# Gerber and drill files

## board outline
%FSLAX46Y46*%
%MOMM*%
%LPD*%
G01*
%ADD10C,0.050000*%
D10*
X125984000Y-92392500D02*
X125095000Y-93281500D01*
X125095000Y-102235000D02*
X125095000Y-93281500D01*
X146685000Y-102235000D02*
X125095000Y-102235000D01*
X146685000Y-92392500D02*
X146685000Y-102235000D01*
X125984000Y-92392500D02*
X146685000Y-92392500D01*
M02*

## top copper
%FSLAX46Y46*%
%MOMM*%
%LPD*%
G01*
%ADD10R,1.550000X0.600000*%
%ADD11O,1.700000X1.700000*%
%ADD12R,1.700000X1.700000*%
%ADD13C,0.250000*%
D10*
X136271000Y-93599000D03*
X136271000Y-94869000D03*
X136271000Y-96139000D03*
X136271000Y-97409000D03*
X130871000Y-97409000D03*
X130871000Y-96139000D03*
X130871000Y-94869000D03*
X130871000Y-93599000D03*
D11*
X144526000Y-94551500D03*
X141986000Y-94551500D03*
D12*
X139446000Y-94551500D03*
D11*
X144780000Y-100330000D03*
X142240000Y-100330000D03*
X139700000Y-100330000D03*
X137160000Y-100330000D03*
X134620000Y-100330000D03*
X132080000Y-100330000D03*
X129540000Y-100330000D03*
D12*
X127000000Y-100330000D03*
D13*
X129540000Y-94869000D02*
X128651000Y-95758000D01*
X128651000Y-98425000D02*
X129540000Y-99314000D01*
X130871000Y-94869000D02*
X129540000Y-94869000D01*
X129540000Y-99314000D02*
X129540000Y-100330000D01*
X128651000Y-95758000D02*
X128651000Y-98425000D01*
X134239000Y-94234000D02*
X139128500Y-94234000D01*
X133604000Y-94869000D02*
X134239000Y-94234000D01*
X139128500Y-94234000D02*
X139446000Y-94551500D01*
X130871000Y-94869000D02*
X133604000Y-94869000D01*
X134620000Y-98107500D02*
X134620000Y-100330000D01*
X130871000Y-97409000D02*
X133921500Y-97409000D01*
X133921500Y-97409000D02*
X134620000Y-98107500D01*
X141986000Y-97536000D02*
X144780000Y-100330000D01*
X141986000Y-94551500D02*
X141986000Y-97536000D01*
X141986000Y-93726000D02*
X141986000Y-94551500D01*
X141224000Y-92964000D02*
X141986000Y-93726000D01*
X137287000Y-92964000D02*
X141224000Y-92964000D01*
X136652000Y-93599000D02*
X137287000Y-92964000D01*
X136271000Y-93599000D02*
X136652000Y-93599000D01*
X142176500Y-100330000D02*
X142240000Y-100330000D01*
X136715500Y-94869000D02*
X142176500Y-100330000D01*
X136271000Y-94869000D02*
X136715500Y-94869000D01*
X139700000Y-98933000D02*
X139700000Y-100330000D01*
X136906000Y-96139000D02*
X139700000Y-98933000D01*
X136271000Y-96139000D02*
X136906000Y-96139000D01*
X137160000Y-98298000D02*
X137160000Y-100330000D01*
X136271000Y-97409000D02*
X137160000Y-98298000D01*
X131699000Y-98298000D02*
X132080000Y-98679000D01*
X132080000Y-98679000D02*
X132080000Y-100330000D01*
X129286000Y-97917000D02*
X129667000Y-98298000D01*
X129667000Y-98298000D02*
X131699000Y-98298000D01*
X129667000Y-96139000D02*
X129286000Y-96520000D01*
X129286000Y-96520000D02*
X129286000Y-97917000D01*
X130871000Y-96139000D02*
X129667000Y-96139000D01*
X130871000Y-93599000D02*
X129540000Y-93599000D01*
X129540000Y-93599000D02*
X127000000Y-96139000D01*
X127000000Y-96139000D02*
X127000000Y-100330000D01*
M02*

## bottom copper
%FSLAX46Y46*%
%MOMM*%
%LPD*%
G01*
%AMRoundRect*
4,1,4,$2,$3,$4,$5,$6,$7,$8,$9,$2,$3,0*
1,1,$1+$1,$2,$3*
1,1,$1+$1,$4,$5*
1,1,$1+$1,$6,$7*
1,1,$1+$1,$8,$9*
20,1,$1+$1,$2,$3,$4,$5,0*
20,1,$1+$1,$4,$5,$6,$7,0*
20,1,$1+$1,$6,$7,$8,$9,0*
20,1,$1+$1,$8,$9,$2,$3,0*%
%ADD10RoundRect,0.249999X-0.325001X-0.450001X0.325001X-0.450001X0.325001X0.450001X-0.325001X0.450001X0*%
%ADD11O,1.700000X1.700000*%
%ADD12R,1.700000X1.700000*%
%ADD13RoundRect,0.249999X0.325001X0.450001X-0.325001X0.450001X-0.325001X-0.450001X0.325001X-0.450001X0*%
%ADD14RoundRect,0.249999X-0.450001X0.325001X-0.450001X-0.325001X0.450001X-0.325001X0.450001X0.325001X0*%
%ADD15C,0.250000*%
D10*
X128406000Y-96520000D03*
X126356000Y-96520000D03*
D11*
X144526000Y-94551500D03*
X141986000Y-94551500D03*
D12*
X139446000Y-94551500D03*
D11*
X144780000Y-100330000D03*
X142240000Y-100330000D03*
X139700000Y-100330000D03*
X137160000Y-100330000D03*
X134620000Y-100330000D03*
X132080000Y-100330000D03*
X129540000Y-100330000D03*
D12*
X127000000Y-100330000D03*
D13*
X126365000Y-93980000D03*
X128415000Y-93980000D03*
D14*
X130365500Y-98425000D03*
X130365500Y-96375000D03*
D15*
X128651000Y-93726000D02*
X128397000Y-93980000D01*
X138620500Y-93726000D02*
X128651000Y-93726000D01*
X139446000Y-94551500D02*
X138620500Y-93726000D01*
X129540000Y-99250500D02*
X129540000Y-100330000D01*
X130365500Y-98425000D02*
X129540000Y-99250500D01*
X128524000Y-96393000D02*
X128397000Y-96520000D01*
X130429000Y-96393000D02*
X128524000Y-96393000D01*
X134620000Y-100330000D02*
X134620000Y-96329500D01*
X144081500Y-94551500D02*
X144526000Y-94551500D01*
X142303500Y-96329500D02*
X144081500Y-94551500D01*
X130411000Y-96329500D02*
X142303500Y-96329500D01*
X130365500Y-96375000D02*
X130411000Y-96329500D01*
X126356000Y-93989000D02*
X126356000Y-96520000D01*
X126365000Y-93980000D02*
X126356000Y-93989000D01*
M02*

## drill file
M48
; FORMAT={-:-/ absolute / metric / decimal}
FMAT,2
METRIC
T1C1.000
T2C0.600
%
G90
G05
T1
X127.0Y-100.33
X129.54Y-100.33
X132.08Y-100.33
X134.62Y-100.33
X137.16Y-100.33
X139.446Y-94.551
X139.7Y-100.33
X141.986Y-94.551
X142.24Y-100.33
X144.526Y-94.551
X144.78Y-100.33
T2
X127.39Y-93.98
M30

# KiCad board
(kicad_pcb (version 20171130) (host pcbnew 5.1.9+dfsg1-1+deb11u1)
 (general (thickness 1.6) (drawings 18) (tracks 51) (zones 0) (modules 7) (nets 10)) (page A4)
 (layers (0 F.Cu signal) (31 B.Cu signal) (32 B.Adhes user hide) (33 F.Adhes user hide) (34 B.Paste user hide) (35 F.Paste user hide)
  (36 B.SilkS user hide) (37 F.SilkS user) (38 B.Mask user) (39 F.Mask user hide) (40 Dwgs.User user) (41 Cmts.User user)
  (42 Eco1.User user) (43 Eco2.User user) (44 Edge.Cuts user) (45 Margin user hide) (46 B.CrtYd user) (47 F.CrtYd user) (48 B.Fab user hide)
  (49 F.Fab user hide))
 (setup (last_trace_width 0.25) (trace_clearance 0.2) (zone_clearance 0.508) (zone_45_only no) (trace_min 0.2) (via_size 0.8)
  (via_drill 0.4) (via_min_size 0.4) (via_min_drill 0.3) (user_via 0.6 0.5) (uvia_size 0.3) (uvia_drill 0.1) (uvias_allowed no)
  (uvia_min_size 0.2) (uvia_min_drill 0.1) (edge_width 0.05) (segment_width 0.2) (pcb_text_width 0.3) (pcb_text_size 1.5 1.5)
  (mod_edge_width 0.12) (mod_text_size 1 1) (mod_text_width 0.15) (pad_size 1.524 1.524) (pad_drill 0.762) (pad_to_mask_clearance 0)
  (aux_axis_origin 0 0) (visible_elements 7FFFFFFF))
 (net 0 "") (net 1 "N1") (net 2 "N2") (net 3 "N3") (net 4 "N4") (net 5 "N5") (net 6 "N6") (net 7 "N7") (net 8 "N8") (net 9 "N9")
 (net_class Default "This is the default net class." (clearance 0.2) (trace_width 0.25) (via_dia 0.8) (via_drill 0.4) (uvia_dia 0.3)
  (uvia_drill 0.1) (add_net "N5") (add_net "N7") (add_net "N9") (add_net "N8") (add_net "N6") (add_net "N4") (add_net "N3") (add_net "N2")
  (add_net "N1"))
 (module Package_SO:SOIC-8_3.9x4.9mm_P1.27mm (layer F.Cu) (at 133.571 95.504)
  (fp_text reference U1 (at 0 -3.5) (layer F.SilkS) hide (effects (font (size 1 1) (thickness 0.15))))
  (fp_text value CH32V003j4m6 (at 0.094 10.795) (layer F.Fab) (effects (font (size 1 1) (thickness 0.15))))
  (pad 8 smd rect (at 2.7 -1.905) (size 1.55 0.6) (layers F.Cu F.Paste F.Mask) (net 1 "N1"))
  (pad 7 smd rect (at 2.7 -0.635) (size 1.55 0.6) (layers F.Cu F.Paste F.Mask) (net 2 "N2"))
  (pad 6 smd rect (at 2.7 0.635) (size 1.55 0.6) (layers F.Cu F.Paste F.Mask) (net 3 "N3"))
  (pad 5 smd rect (at 2.7 1.905) (size 1.55 0.6) (layers F.Cu F.Paste F.Mask) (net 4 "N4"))
  (pad 4 smd rect (at -2.7 1.905) (size 1.55 0.6) (layers F.Cu F.Paste F.Mask) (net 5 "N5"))
  (pad 3 smd rect (at -2.7 0.635) (size 1.55 0.6) (layers F.Cu F.Paste F.Mask) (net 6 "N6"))
  (pad 2 smd rect (at -2.7 -0.635) (size 1.55 0.6) (layers F.Cu F.Paste F.Mask) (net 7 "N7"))
  (pad 1 smd rect (at -2.7 -1.905) (size 1.55 0.6) (layers F.Cu F.Paste F.Mask) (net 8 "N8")))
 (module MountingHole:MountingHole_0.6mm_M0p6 (layer F.Cu) (at 127.39 93.98)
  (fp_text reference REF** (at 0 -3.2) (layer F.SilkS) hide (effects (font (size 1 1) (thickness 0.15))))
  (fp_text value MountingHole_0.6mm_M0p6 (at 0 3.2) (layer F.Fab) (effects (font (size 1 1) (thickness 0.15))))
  (pad "" np_thru_hole circle (at 0 0) (size 0.6 0.6) (drill 0.6) (layers *.Cu *.Mask)))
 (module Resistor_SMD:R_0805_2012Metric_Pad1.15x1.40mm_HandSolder (layer B.Cu) (at 127.381 96.52)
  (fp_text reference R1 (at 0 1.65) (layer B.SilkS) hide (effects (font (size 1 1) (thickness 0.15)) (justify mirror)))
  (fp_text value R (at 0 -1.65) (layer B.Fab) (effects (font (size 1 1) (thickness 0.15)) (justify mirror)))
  (pad 2 smd roundrect (at 1.025 0) (size 1.15 1.4) (layers B.Cu B.Paste B.Mask) (roundrect_rratio 0.2173904347826087) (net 5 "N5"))
  (pad 1 smd roundrect (at -1.025 0) (size 1.15 1.4) (layers B.Cu B.Paste B.Mask) (roundrect_rratio 0.2173904347826087) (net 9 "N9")))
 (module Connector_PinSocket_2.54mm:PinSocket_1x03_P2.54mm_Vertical (layer F.Cu) (at 139.446 94.5515 90)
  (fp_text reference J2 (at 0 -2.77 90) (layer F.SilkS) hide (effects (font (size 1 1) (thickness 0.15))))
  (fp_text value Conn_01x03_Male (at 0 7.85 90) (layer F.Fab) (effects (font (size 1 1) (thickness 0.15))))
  (pad 3 thru_hole oval (at 0 5.08 90) (size 1.7 1.7) (drill 1) (layers *.Cu *.Mask) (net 5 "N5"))
  (pad 2 thru_hole oval (at 0 2.54 90) (size 1.7 1.7) (drill 1) (layers *.Cu *.Mask) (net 1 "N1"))
  (pad 1 thru_hole rect (at 0 0 90) (size 1.7 1.7) (drill 1) (layers *.Cu *.Mask) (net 7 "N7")))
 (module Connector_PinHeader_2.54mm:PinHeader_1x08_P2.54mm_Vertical (layer F.Cu) (at 127 100.33 90)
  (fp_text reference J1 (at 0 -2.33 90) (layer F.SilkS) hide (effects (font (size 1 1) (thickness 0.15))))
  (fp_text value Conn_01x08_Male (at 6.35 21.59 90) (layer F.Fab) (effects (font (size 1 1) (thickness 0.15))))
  (pad 8 thru_hole oval (at 0 17.78 90) (size 1.7 1.7) (drill 1) (layers *.Cu *.Mask) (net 1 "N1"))
  (pad 7 thru_hole oval (at 0 15.24 90) (size 1.7 1.7) (drill 1) (layers *.Cu *.Mask) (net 2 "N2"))
  (pad 6 thru_hole oval (at 0 12.7 90) (size 1.7 1.7) (drill 1) (layers *.Cu *.Mask) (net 3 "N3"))
  (pad 5 thru_hole oval (at 0 10.16 90) (size 1.7 1.7) (drill 1) (layers *.Cu *.Mask) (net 4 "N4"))
  (pad 4 thru_hole oval (at 0 7.62 90) (size 1.7 1.7) (drill 1) (layers *.Cu *.Mask) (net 5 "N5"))
  (pad 3 thru_hole oval (at 0 5.08 90) (size 1.7 1.7) (drill 1) (layers *.Cu *.Mask) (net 6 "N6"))
  (pad 2 thru_hole oval (at 0 2.54 90) (size 1.7 1.7) (drill 1) (layers *.Cu *.Mask) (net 7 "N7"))
  (pad 1 thru_hole rect (at 0 0 90) (size 1.7 1.7) (drill 1) (layers *.Cu *.Mask) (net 8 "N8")))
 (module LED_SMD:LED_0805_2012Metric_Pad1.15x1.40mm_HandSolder (layer B.Cu) (at 127.39 93.98 180)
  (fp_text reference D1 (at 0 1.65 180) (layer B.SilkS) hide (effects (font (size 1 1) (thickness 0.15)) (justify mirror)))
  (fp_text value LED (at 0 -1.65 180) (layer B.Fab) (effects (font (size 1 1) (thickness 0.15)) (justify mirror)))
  (pad 2 smd roundrect (at 1.025 0 180) (size 1.15 1.4) (layers B.Cu B.Paste B.Mask) (roundrect_rratio 0.2173904347826087) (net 9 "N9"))
  (pad 1 smd roundrect (at -1.025 0 180) (size 1.15 1.4) (layers B.Cu B.Paste B.Mask) (roundrect_rratio 0.2173904347826087) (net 7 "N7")))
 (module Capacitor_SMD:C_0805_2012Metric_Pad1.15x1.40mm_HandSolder (layer B.Cu) (at 130.3655 97.4 270)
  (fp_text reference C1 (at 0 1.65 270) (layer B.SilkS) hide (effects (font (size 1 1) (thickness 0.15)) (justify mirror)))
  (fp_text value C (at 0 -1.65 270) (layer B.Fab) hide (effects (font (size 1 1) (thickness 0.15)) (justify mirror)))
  (pad 2 smd roundrect (at 1.025 0 270) (size 1.15 1.4) (layers B.Cu B.Paste B.Mask) (roundrect_rratio 0.2173904347826087) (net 7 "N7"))
  (pad 1 smd roundrect (at -1.025 0 270) (size 1.15 1.4) (layers B.Cu B.Paste B.Mask) (roundrect_rratio 0.2173904347826087) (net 5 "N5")))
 (gr_line (start 125.984 92.3925) (end 125.095 93.2815) (layer Edge.Cuts) (width 0.05))
 (gr_line (start 125.095 102.235) (end 125.095 93.2815) (layer Edge.Cuts) (width 0.05))
 (gr_line (start 146.685 102.235) (end 125.095 102.235) (layer Edge.Cuts) (width 0.05))
 (gr_line (start 146.685 92.3925) (end 146.685 102.235) (layer Edge.Cuts) (width 0.05))
 (gr_line (start 125.984 92.3925) (end 146.685 92.3925) (layer Edge.Cuts) (width 0.05))
 (segment (start 129.54 94.869) (end 128.651 95.758) (width 0.25) (layer F.Cu) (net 7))
 (segment (start 128.651 98.425) (end 129.54 99.314) (width 0.25) (layer F.Cu) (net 7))
 (segment (start 130.871 94.869) (end 129.54 94.869) (width 0.25) (layer F.Cu) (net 7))
 (segment (start 129.54 99.314) (end 129.54 100.33) (width 0.25) (layer F.Cu) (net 7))
 (segment (start 128.651 95.758) (end 128.651 98.425) (width 0.25) (layer F.Cu) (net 7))
 (segment (start 128.651 93.726) (end 128.397 93.98) (width 0.25) (layer B.Cu) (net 7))
 (segment (start 138.6205 93.726) (end 128.651 93.726) (width 0.25) (layer B.Cu) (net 7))
 (segment (start 139.446 94.5515) (end 138.6205 93.726) (width 0.25) (layer B.Cu) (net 7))
 (segment (start 134.239 94.234) (end 139.1285 94.234) (width 0.25) (layer F.Cu) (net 7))
 (segment (start 133.604 94.869) (end 134.239 94.234) (width 0.25) (layer F.Cu) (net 7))
 (segment (start 139.1285 94.234) (end 139.446 94.5515) (width 0.25) (layer F.Cu) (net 7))
 (segment (start 130.871 94.869) (end 133.604 94.869) (width 0.25) (layer F.Cu) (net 7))
 (segment (start 129.54 99.2505) (end 129.54 100.33) (width 0.25) (layer B.Cu) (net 7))
 (segment (start 130.3655 98.425) (end 129.54 99.2505) (width 0.25) (layer B.Cu) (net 7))
 (segment (start 134.62 98.1075) (end 134.62 100.33) (width 0.25) (layer F.Cu) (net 5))
 (segment (start 130.871 97.409) (end 133.9215 97.409) (width 0.25) (layer F.Cu) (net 5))
 (segment (start 133.9215 97.409) (end 134.62 98.1075) (width 0.25) (layer F.Cu) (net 5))
 (segment (start 128.524 96.393) (end 128.397 96.52) (width 0.25) (layer B.Cu) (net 5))
 (segment (start 130.429 96.393) (end 128.524 96.393) (width 0.25) (layer B.Cu) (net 5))
 (segment (start 134.62 100.33) (end 134.62 96.3295) (width 0.25) (layer B.Cu) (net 5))
 (segment (start 144.0815 94.5515) (end 144.526 94.5515) (width 0.25) (layer B.Cu) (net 5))
 (segment (start 142.3035 96.3295) (end 144.0815 94.5515) (width 0.25) (layer B.Cu) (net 5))
 (segment (start 130.411 96.3295) (end 142.3035 96.3295) (width 0.25) (layer B.Cu) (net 5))
 (segment (start 130.3655 96.375) (end 130.411 96.3295) (width 0.25) (layer B.Cu) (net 5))
 (segment (start 126.356 93.989) (end 126.356 96.52) (width 0.25) (layer B.Cu) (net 9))
 (segment (start 126.365 93.98) (end 126.356 93.989) (width 0.25) (layer B.Cu) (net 9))
 (segment (start 141.986 97.536) (end 144.78 100.33) (width 0.25) (layer F.Cu) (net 1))
 (segment (start 141.986 94.5515) (end 141.986 97.536) (width 0.25) (layer F.Cu) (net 1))
 (segment (start 141.986 93.726) (end 141.986 94.5515) (width 0.25) (layer F.Cu) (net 1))
 (segment (start 141.224 92.964) (end 141.986 93.726) (width 0.25) (layer F.Cu) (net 1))
 (segment (start 137.287 92.964) (end 141.224 92.964) (width 0.25) (layer F.Cu) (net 1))
 (segment (start 136.652 93.599) (end 137.287 92.964) (width 0.25) (layer F.Cu) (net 1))
 (segment (start 136.271 93.599) (end 136.652 93.599) (width 0.25) (layer F.Cu) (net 1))
 (segment (start 142.1765 100.33) (end 142.24 100.33) (width 0.25) (layer F.Cu) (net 2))
 (segment (start 136.7155 94.869) (end 142.1765 100.33) (width 0.25) (layer F.Cu) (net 2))
 (segment (start 136.271 94.869) (end 136.7155 94.869) (width 0.25) (layer F.Cu) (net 2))
 (segment (start 139.7 98.933) (end 139.7 100.33) (width 0.25) (layer F.Cu) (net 3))
 (segment (start 136.906 96.139) (end 139.7 98.933) (width 0.25) (layer F.Cu) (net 3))
 (segment (start 136.271 96.139) (end 136.906 96.139) (width 0.25) (layer F.Cu) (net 3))
 (segment (start 137.16 98.298) (end 137.16 100.33) (width 0.25) (layer F.Cu) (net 4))
 (segment (start 136.271 97.409) (end 137.16 98.298) (width 0.25) (layer F.Cu) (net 4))
 (segment (start 131.699 98.298) (end 132.08 98.679) (width 0.25) (layer F.Cu) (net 6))
 (segment (start 132.08 98.679) (end 132.08 100.33) (width 0.25) (layer F.Cu) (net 6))
 (segment (start 129.286 97.917) (end 129.667 98.298) (width 0.25) (layer F.Cu) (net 6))
 (segment (start 129.667 98.298) (end 131.699 98.298) (width 0.25) (layer F.Cu) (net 6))
 (segment (start 129.667 96.139) (end 129.286 96.52) (width 0.25) (layer F.Cu) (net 6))
 (segment (start 129.286 96.52) (end 129.286 97.917) (width 0.25) (layer F.Cu) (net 6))
 (segment (start 130.871 96.139) (end 129.667 96.139) (width 0.25) (layer F.Cu) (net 6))
 (segment (start 130.871 93.599) (end 129.54 93.599) (width 0.25) (layer F.Cu) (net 8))
 (segment (start 129.54 93.599) (end 127 96.139) (width 0.25) (layer F.Cu) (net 8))
 (segment (start 127 96.139) (end 127 100.33) (width 0.25) (layer F.Cu) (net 8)))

